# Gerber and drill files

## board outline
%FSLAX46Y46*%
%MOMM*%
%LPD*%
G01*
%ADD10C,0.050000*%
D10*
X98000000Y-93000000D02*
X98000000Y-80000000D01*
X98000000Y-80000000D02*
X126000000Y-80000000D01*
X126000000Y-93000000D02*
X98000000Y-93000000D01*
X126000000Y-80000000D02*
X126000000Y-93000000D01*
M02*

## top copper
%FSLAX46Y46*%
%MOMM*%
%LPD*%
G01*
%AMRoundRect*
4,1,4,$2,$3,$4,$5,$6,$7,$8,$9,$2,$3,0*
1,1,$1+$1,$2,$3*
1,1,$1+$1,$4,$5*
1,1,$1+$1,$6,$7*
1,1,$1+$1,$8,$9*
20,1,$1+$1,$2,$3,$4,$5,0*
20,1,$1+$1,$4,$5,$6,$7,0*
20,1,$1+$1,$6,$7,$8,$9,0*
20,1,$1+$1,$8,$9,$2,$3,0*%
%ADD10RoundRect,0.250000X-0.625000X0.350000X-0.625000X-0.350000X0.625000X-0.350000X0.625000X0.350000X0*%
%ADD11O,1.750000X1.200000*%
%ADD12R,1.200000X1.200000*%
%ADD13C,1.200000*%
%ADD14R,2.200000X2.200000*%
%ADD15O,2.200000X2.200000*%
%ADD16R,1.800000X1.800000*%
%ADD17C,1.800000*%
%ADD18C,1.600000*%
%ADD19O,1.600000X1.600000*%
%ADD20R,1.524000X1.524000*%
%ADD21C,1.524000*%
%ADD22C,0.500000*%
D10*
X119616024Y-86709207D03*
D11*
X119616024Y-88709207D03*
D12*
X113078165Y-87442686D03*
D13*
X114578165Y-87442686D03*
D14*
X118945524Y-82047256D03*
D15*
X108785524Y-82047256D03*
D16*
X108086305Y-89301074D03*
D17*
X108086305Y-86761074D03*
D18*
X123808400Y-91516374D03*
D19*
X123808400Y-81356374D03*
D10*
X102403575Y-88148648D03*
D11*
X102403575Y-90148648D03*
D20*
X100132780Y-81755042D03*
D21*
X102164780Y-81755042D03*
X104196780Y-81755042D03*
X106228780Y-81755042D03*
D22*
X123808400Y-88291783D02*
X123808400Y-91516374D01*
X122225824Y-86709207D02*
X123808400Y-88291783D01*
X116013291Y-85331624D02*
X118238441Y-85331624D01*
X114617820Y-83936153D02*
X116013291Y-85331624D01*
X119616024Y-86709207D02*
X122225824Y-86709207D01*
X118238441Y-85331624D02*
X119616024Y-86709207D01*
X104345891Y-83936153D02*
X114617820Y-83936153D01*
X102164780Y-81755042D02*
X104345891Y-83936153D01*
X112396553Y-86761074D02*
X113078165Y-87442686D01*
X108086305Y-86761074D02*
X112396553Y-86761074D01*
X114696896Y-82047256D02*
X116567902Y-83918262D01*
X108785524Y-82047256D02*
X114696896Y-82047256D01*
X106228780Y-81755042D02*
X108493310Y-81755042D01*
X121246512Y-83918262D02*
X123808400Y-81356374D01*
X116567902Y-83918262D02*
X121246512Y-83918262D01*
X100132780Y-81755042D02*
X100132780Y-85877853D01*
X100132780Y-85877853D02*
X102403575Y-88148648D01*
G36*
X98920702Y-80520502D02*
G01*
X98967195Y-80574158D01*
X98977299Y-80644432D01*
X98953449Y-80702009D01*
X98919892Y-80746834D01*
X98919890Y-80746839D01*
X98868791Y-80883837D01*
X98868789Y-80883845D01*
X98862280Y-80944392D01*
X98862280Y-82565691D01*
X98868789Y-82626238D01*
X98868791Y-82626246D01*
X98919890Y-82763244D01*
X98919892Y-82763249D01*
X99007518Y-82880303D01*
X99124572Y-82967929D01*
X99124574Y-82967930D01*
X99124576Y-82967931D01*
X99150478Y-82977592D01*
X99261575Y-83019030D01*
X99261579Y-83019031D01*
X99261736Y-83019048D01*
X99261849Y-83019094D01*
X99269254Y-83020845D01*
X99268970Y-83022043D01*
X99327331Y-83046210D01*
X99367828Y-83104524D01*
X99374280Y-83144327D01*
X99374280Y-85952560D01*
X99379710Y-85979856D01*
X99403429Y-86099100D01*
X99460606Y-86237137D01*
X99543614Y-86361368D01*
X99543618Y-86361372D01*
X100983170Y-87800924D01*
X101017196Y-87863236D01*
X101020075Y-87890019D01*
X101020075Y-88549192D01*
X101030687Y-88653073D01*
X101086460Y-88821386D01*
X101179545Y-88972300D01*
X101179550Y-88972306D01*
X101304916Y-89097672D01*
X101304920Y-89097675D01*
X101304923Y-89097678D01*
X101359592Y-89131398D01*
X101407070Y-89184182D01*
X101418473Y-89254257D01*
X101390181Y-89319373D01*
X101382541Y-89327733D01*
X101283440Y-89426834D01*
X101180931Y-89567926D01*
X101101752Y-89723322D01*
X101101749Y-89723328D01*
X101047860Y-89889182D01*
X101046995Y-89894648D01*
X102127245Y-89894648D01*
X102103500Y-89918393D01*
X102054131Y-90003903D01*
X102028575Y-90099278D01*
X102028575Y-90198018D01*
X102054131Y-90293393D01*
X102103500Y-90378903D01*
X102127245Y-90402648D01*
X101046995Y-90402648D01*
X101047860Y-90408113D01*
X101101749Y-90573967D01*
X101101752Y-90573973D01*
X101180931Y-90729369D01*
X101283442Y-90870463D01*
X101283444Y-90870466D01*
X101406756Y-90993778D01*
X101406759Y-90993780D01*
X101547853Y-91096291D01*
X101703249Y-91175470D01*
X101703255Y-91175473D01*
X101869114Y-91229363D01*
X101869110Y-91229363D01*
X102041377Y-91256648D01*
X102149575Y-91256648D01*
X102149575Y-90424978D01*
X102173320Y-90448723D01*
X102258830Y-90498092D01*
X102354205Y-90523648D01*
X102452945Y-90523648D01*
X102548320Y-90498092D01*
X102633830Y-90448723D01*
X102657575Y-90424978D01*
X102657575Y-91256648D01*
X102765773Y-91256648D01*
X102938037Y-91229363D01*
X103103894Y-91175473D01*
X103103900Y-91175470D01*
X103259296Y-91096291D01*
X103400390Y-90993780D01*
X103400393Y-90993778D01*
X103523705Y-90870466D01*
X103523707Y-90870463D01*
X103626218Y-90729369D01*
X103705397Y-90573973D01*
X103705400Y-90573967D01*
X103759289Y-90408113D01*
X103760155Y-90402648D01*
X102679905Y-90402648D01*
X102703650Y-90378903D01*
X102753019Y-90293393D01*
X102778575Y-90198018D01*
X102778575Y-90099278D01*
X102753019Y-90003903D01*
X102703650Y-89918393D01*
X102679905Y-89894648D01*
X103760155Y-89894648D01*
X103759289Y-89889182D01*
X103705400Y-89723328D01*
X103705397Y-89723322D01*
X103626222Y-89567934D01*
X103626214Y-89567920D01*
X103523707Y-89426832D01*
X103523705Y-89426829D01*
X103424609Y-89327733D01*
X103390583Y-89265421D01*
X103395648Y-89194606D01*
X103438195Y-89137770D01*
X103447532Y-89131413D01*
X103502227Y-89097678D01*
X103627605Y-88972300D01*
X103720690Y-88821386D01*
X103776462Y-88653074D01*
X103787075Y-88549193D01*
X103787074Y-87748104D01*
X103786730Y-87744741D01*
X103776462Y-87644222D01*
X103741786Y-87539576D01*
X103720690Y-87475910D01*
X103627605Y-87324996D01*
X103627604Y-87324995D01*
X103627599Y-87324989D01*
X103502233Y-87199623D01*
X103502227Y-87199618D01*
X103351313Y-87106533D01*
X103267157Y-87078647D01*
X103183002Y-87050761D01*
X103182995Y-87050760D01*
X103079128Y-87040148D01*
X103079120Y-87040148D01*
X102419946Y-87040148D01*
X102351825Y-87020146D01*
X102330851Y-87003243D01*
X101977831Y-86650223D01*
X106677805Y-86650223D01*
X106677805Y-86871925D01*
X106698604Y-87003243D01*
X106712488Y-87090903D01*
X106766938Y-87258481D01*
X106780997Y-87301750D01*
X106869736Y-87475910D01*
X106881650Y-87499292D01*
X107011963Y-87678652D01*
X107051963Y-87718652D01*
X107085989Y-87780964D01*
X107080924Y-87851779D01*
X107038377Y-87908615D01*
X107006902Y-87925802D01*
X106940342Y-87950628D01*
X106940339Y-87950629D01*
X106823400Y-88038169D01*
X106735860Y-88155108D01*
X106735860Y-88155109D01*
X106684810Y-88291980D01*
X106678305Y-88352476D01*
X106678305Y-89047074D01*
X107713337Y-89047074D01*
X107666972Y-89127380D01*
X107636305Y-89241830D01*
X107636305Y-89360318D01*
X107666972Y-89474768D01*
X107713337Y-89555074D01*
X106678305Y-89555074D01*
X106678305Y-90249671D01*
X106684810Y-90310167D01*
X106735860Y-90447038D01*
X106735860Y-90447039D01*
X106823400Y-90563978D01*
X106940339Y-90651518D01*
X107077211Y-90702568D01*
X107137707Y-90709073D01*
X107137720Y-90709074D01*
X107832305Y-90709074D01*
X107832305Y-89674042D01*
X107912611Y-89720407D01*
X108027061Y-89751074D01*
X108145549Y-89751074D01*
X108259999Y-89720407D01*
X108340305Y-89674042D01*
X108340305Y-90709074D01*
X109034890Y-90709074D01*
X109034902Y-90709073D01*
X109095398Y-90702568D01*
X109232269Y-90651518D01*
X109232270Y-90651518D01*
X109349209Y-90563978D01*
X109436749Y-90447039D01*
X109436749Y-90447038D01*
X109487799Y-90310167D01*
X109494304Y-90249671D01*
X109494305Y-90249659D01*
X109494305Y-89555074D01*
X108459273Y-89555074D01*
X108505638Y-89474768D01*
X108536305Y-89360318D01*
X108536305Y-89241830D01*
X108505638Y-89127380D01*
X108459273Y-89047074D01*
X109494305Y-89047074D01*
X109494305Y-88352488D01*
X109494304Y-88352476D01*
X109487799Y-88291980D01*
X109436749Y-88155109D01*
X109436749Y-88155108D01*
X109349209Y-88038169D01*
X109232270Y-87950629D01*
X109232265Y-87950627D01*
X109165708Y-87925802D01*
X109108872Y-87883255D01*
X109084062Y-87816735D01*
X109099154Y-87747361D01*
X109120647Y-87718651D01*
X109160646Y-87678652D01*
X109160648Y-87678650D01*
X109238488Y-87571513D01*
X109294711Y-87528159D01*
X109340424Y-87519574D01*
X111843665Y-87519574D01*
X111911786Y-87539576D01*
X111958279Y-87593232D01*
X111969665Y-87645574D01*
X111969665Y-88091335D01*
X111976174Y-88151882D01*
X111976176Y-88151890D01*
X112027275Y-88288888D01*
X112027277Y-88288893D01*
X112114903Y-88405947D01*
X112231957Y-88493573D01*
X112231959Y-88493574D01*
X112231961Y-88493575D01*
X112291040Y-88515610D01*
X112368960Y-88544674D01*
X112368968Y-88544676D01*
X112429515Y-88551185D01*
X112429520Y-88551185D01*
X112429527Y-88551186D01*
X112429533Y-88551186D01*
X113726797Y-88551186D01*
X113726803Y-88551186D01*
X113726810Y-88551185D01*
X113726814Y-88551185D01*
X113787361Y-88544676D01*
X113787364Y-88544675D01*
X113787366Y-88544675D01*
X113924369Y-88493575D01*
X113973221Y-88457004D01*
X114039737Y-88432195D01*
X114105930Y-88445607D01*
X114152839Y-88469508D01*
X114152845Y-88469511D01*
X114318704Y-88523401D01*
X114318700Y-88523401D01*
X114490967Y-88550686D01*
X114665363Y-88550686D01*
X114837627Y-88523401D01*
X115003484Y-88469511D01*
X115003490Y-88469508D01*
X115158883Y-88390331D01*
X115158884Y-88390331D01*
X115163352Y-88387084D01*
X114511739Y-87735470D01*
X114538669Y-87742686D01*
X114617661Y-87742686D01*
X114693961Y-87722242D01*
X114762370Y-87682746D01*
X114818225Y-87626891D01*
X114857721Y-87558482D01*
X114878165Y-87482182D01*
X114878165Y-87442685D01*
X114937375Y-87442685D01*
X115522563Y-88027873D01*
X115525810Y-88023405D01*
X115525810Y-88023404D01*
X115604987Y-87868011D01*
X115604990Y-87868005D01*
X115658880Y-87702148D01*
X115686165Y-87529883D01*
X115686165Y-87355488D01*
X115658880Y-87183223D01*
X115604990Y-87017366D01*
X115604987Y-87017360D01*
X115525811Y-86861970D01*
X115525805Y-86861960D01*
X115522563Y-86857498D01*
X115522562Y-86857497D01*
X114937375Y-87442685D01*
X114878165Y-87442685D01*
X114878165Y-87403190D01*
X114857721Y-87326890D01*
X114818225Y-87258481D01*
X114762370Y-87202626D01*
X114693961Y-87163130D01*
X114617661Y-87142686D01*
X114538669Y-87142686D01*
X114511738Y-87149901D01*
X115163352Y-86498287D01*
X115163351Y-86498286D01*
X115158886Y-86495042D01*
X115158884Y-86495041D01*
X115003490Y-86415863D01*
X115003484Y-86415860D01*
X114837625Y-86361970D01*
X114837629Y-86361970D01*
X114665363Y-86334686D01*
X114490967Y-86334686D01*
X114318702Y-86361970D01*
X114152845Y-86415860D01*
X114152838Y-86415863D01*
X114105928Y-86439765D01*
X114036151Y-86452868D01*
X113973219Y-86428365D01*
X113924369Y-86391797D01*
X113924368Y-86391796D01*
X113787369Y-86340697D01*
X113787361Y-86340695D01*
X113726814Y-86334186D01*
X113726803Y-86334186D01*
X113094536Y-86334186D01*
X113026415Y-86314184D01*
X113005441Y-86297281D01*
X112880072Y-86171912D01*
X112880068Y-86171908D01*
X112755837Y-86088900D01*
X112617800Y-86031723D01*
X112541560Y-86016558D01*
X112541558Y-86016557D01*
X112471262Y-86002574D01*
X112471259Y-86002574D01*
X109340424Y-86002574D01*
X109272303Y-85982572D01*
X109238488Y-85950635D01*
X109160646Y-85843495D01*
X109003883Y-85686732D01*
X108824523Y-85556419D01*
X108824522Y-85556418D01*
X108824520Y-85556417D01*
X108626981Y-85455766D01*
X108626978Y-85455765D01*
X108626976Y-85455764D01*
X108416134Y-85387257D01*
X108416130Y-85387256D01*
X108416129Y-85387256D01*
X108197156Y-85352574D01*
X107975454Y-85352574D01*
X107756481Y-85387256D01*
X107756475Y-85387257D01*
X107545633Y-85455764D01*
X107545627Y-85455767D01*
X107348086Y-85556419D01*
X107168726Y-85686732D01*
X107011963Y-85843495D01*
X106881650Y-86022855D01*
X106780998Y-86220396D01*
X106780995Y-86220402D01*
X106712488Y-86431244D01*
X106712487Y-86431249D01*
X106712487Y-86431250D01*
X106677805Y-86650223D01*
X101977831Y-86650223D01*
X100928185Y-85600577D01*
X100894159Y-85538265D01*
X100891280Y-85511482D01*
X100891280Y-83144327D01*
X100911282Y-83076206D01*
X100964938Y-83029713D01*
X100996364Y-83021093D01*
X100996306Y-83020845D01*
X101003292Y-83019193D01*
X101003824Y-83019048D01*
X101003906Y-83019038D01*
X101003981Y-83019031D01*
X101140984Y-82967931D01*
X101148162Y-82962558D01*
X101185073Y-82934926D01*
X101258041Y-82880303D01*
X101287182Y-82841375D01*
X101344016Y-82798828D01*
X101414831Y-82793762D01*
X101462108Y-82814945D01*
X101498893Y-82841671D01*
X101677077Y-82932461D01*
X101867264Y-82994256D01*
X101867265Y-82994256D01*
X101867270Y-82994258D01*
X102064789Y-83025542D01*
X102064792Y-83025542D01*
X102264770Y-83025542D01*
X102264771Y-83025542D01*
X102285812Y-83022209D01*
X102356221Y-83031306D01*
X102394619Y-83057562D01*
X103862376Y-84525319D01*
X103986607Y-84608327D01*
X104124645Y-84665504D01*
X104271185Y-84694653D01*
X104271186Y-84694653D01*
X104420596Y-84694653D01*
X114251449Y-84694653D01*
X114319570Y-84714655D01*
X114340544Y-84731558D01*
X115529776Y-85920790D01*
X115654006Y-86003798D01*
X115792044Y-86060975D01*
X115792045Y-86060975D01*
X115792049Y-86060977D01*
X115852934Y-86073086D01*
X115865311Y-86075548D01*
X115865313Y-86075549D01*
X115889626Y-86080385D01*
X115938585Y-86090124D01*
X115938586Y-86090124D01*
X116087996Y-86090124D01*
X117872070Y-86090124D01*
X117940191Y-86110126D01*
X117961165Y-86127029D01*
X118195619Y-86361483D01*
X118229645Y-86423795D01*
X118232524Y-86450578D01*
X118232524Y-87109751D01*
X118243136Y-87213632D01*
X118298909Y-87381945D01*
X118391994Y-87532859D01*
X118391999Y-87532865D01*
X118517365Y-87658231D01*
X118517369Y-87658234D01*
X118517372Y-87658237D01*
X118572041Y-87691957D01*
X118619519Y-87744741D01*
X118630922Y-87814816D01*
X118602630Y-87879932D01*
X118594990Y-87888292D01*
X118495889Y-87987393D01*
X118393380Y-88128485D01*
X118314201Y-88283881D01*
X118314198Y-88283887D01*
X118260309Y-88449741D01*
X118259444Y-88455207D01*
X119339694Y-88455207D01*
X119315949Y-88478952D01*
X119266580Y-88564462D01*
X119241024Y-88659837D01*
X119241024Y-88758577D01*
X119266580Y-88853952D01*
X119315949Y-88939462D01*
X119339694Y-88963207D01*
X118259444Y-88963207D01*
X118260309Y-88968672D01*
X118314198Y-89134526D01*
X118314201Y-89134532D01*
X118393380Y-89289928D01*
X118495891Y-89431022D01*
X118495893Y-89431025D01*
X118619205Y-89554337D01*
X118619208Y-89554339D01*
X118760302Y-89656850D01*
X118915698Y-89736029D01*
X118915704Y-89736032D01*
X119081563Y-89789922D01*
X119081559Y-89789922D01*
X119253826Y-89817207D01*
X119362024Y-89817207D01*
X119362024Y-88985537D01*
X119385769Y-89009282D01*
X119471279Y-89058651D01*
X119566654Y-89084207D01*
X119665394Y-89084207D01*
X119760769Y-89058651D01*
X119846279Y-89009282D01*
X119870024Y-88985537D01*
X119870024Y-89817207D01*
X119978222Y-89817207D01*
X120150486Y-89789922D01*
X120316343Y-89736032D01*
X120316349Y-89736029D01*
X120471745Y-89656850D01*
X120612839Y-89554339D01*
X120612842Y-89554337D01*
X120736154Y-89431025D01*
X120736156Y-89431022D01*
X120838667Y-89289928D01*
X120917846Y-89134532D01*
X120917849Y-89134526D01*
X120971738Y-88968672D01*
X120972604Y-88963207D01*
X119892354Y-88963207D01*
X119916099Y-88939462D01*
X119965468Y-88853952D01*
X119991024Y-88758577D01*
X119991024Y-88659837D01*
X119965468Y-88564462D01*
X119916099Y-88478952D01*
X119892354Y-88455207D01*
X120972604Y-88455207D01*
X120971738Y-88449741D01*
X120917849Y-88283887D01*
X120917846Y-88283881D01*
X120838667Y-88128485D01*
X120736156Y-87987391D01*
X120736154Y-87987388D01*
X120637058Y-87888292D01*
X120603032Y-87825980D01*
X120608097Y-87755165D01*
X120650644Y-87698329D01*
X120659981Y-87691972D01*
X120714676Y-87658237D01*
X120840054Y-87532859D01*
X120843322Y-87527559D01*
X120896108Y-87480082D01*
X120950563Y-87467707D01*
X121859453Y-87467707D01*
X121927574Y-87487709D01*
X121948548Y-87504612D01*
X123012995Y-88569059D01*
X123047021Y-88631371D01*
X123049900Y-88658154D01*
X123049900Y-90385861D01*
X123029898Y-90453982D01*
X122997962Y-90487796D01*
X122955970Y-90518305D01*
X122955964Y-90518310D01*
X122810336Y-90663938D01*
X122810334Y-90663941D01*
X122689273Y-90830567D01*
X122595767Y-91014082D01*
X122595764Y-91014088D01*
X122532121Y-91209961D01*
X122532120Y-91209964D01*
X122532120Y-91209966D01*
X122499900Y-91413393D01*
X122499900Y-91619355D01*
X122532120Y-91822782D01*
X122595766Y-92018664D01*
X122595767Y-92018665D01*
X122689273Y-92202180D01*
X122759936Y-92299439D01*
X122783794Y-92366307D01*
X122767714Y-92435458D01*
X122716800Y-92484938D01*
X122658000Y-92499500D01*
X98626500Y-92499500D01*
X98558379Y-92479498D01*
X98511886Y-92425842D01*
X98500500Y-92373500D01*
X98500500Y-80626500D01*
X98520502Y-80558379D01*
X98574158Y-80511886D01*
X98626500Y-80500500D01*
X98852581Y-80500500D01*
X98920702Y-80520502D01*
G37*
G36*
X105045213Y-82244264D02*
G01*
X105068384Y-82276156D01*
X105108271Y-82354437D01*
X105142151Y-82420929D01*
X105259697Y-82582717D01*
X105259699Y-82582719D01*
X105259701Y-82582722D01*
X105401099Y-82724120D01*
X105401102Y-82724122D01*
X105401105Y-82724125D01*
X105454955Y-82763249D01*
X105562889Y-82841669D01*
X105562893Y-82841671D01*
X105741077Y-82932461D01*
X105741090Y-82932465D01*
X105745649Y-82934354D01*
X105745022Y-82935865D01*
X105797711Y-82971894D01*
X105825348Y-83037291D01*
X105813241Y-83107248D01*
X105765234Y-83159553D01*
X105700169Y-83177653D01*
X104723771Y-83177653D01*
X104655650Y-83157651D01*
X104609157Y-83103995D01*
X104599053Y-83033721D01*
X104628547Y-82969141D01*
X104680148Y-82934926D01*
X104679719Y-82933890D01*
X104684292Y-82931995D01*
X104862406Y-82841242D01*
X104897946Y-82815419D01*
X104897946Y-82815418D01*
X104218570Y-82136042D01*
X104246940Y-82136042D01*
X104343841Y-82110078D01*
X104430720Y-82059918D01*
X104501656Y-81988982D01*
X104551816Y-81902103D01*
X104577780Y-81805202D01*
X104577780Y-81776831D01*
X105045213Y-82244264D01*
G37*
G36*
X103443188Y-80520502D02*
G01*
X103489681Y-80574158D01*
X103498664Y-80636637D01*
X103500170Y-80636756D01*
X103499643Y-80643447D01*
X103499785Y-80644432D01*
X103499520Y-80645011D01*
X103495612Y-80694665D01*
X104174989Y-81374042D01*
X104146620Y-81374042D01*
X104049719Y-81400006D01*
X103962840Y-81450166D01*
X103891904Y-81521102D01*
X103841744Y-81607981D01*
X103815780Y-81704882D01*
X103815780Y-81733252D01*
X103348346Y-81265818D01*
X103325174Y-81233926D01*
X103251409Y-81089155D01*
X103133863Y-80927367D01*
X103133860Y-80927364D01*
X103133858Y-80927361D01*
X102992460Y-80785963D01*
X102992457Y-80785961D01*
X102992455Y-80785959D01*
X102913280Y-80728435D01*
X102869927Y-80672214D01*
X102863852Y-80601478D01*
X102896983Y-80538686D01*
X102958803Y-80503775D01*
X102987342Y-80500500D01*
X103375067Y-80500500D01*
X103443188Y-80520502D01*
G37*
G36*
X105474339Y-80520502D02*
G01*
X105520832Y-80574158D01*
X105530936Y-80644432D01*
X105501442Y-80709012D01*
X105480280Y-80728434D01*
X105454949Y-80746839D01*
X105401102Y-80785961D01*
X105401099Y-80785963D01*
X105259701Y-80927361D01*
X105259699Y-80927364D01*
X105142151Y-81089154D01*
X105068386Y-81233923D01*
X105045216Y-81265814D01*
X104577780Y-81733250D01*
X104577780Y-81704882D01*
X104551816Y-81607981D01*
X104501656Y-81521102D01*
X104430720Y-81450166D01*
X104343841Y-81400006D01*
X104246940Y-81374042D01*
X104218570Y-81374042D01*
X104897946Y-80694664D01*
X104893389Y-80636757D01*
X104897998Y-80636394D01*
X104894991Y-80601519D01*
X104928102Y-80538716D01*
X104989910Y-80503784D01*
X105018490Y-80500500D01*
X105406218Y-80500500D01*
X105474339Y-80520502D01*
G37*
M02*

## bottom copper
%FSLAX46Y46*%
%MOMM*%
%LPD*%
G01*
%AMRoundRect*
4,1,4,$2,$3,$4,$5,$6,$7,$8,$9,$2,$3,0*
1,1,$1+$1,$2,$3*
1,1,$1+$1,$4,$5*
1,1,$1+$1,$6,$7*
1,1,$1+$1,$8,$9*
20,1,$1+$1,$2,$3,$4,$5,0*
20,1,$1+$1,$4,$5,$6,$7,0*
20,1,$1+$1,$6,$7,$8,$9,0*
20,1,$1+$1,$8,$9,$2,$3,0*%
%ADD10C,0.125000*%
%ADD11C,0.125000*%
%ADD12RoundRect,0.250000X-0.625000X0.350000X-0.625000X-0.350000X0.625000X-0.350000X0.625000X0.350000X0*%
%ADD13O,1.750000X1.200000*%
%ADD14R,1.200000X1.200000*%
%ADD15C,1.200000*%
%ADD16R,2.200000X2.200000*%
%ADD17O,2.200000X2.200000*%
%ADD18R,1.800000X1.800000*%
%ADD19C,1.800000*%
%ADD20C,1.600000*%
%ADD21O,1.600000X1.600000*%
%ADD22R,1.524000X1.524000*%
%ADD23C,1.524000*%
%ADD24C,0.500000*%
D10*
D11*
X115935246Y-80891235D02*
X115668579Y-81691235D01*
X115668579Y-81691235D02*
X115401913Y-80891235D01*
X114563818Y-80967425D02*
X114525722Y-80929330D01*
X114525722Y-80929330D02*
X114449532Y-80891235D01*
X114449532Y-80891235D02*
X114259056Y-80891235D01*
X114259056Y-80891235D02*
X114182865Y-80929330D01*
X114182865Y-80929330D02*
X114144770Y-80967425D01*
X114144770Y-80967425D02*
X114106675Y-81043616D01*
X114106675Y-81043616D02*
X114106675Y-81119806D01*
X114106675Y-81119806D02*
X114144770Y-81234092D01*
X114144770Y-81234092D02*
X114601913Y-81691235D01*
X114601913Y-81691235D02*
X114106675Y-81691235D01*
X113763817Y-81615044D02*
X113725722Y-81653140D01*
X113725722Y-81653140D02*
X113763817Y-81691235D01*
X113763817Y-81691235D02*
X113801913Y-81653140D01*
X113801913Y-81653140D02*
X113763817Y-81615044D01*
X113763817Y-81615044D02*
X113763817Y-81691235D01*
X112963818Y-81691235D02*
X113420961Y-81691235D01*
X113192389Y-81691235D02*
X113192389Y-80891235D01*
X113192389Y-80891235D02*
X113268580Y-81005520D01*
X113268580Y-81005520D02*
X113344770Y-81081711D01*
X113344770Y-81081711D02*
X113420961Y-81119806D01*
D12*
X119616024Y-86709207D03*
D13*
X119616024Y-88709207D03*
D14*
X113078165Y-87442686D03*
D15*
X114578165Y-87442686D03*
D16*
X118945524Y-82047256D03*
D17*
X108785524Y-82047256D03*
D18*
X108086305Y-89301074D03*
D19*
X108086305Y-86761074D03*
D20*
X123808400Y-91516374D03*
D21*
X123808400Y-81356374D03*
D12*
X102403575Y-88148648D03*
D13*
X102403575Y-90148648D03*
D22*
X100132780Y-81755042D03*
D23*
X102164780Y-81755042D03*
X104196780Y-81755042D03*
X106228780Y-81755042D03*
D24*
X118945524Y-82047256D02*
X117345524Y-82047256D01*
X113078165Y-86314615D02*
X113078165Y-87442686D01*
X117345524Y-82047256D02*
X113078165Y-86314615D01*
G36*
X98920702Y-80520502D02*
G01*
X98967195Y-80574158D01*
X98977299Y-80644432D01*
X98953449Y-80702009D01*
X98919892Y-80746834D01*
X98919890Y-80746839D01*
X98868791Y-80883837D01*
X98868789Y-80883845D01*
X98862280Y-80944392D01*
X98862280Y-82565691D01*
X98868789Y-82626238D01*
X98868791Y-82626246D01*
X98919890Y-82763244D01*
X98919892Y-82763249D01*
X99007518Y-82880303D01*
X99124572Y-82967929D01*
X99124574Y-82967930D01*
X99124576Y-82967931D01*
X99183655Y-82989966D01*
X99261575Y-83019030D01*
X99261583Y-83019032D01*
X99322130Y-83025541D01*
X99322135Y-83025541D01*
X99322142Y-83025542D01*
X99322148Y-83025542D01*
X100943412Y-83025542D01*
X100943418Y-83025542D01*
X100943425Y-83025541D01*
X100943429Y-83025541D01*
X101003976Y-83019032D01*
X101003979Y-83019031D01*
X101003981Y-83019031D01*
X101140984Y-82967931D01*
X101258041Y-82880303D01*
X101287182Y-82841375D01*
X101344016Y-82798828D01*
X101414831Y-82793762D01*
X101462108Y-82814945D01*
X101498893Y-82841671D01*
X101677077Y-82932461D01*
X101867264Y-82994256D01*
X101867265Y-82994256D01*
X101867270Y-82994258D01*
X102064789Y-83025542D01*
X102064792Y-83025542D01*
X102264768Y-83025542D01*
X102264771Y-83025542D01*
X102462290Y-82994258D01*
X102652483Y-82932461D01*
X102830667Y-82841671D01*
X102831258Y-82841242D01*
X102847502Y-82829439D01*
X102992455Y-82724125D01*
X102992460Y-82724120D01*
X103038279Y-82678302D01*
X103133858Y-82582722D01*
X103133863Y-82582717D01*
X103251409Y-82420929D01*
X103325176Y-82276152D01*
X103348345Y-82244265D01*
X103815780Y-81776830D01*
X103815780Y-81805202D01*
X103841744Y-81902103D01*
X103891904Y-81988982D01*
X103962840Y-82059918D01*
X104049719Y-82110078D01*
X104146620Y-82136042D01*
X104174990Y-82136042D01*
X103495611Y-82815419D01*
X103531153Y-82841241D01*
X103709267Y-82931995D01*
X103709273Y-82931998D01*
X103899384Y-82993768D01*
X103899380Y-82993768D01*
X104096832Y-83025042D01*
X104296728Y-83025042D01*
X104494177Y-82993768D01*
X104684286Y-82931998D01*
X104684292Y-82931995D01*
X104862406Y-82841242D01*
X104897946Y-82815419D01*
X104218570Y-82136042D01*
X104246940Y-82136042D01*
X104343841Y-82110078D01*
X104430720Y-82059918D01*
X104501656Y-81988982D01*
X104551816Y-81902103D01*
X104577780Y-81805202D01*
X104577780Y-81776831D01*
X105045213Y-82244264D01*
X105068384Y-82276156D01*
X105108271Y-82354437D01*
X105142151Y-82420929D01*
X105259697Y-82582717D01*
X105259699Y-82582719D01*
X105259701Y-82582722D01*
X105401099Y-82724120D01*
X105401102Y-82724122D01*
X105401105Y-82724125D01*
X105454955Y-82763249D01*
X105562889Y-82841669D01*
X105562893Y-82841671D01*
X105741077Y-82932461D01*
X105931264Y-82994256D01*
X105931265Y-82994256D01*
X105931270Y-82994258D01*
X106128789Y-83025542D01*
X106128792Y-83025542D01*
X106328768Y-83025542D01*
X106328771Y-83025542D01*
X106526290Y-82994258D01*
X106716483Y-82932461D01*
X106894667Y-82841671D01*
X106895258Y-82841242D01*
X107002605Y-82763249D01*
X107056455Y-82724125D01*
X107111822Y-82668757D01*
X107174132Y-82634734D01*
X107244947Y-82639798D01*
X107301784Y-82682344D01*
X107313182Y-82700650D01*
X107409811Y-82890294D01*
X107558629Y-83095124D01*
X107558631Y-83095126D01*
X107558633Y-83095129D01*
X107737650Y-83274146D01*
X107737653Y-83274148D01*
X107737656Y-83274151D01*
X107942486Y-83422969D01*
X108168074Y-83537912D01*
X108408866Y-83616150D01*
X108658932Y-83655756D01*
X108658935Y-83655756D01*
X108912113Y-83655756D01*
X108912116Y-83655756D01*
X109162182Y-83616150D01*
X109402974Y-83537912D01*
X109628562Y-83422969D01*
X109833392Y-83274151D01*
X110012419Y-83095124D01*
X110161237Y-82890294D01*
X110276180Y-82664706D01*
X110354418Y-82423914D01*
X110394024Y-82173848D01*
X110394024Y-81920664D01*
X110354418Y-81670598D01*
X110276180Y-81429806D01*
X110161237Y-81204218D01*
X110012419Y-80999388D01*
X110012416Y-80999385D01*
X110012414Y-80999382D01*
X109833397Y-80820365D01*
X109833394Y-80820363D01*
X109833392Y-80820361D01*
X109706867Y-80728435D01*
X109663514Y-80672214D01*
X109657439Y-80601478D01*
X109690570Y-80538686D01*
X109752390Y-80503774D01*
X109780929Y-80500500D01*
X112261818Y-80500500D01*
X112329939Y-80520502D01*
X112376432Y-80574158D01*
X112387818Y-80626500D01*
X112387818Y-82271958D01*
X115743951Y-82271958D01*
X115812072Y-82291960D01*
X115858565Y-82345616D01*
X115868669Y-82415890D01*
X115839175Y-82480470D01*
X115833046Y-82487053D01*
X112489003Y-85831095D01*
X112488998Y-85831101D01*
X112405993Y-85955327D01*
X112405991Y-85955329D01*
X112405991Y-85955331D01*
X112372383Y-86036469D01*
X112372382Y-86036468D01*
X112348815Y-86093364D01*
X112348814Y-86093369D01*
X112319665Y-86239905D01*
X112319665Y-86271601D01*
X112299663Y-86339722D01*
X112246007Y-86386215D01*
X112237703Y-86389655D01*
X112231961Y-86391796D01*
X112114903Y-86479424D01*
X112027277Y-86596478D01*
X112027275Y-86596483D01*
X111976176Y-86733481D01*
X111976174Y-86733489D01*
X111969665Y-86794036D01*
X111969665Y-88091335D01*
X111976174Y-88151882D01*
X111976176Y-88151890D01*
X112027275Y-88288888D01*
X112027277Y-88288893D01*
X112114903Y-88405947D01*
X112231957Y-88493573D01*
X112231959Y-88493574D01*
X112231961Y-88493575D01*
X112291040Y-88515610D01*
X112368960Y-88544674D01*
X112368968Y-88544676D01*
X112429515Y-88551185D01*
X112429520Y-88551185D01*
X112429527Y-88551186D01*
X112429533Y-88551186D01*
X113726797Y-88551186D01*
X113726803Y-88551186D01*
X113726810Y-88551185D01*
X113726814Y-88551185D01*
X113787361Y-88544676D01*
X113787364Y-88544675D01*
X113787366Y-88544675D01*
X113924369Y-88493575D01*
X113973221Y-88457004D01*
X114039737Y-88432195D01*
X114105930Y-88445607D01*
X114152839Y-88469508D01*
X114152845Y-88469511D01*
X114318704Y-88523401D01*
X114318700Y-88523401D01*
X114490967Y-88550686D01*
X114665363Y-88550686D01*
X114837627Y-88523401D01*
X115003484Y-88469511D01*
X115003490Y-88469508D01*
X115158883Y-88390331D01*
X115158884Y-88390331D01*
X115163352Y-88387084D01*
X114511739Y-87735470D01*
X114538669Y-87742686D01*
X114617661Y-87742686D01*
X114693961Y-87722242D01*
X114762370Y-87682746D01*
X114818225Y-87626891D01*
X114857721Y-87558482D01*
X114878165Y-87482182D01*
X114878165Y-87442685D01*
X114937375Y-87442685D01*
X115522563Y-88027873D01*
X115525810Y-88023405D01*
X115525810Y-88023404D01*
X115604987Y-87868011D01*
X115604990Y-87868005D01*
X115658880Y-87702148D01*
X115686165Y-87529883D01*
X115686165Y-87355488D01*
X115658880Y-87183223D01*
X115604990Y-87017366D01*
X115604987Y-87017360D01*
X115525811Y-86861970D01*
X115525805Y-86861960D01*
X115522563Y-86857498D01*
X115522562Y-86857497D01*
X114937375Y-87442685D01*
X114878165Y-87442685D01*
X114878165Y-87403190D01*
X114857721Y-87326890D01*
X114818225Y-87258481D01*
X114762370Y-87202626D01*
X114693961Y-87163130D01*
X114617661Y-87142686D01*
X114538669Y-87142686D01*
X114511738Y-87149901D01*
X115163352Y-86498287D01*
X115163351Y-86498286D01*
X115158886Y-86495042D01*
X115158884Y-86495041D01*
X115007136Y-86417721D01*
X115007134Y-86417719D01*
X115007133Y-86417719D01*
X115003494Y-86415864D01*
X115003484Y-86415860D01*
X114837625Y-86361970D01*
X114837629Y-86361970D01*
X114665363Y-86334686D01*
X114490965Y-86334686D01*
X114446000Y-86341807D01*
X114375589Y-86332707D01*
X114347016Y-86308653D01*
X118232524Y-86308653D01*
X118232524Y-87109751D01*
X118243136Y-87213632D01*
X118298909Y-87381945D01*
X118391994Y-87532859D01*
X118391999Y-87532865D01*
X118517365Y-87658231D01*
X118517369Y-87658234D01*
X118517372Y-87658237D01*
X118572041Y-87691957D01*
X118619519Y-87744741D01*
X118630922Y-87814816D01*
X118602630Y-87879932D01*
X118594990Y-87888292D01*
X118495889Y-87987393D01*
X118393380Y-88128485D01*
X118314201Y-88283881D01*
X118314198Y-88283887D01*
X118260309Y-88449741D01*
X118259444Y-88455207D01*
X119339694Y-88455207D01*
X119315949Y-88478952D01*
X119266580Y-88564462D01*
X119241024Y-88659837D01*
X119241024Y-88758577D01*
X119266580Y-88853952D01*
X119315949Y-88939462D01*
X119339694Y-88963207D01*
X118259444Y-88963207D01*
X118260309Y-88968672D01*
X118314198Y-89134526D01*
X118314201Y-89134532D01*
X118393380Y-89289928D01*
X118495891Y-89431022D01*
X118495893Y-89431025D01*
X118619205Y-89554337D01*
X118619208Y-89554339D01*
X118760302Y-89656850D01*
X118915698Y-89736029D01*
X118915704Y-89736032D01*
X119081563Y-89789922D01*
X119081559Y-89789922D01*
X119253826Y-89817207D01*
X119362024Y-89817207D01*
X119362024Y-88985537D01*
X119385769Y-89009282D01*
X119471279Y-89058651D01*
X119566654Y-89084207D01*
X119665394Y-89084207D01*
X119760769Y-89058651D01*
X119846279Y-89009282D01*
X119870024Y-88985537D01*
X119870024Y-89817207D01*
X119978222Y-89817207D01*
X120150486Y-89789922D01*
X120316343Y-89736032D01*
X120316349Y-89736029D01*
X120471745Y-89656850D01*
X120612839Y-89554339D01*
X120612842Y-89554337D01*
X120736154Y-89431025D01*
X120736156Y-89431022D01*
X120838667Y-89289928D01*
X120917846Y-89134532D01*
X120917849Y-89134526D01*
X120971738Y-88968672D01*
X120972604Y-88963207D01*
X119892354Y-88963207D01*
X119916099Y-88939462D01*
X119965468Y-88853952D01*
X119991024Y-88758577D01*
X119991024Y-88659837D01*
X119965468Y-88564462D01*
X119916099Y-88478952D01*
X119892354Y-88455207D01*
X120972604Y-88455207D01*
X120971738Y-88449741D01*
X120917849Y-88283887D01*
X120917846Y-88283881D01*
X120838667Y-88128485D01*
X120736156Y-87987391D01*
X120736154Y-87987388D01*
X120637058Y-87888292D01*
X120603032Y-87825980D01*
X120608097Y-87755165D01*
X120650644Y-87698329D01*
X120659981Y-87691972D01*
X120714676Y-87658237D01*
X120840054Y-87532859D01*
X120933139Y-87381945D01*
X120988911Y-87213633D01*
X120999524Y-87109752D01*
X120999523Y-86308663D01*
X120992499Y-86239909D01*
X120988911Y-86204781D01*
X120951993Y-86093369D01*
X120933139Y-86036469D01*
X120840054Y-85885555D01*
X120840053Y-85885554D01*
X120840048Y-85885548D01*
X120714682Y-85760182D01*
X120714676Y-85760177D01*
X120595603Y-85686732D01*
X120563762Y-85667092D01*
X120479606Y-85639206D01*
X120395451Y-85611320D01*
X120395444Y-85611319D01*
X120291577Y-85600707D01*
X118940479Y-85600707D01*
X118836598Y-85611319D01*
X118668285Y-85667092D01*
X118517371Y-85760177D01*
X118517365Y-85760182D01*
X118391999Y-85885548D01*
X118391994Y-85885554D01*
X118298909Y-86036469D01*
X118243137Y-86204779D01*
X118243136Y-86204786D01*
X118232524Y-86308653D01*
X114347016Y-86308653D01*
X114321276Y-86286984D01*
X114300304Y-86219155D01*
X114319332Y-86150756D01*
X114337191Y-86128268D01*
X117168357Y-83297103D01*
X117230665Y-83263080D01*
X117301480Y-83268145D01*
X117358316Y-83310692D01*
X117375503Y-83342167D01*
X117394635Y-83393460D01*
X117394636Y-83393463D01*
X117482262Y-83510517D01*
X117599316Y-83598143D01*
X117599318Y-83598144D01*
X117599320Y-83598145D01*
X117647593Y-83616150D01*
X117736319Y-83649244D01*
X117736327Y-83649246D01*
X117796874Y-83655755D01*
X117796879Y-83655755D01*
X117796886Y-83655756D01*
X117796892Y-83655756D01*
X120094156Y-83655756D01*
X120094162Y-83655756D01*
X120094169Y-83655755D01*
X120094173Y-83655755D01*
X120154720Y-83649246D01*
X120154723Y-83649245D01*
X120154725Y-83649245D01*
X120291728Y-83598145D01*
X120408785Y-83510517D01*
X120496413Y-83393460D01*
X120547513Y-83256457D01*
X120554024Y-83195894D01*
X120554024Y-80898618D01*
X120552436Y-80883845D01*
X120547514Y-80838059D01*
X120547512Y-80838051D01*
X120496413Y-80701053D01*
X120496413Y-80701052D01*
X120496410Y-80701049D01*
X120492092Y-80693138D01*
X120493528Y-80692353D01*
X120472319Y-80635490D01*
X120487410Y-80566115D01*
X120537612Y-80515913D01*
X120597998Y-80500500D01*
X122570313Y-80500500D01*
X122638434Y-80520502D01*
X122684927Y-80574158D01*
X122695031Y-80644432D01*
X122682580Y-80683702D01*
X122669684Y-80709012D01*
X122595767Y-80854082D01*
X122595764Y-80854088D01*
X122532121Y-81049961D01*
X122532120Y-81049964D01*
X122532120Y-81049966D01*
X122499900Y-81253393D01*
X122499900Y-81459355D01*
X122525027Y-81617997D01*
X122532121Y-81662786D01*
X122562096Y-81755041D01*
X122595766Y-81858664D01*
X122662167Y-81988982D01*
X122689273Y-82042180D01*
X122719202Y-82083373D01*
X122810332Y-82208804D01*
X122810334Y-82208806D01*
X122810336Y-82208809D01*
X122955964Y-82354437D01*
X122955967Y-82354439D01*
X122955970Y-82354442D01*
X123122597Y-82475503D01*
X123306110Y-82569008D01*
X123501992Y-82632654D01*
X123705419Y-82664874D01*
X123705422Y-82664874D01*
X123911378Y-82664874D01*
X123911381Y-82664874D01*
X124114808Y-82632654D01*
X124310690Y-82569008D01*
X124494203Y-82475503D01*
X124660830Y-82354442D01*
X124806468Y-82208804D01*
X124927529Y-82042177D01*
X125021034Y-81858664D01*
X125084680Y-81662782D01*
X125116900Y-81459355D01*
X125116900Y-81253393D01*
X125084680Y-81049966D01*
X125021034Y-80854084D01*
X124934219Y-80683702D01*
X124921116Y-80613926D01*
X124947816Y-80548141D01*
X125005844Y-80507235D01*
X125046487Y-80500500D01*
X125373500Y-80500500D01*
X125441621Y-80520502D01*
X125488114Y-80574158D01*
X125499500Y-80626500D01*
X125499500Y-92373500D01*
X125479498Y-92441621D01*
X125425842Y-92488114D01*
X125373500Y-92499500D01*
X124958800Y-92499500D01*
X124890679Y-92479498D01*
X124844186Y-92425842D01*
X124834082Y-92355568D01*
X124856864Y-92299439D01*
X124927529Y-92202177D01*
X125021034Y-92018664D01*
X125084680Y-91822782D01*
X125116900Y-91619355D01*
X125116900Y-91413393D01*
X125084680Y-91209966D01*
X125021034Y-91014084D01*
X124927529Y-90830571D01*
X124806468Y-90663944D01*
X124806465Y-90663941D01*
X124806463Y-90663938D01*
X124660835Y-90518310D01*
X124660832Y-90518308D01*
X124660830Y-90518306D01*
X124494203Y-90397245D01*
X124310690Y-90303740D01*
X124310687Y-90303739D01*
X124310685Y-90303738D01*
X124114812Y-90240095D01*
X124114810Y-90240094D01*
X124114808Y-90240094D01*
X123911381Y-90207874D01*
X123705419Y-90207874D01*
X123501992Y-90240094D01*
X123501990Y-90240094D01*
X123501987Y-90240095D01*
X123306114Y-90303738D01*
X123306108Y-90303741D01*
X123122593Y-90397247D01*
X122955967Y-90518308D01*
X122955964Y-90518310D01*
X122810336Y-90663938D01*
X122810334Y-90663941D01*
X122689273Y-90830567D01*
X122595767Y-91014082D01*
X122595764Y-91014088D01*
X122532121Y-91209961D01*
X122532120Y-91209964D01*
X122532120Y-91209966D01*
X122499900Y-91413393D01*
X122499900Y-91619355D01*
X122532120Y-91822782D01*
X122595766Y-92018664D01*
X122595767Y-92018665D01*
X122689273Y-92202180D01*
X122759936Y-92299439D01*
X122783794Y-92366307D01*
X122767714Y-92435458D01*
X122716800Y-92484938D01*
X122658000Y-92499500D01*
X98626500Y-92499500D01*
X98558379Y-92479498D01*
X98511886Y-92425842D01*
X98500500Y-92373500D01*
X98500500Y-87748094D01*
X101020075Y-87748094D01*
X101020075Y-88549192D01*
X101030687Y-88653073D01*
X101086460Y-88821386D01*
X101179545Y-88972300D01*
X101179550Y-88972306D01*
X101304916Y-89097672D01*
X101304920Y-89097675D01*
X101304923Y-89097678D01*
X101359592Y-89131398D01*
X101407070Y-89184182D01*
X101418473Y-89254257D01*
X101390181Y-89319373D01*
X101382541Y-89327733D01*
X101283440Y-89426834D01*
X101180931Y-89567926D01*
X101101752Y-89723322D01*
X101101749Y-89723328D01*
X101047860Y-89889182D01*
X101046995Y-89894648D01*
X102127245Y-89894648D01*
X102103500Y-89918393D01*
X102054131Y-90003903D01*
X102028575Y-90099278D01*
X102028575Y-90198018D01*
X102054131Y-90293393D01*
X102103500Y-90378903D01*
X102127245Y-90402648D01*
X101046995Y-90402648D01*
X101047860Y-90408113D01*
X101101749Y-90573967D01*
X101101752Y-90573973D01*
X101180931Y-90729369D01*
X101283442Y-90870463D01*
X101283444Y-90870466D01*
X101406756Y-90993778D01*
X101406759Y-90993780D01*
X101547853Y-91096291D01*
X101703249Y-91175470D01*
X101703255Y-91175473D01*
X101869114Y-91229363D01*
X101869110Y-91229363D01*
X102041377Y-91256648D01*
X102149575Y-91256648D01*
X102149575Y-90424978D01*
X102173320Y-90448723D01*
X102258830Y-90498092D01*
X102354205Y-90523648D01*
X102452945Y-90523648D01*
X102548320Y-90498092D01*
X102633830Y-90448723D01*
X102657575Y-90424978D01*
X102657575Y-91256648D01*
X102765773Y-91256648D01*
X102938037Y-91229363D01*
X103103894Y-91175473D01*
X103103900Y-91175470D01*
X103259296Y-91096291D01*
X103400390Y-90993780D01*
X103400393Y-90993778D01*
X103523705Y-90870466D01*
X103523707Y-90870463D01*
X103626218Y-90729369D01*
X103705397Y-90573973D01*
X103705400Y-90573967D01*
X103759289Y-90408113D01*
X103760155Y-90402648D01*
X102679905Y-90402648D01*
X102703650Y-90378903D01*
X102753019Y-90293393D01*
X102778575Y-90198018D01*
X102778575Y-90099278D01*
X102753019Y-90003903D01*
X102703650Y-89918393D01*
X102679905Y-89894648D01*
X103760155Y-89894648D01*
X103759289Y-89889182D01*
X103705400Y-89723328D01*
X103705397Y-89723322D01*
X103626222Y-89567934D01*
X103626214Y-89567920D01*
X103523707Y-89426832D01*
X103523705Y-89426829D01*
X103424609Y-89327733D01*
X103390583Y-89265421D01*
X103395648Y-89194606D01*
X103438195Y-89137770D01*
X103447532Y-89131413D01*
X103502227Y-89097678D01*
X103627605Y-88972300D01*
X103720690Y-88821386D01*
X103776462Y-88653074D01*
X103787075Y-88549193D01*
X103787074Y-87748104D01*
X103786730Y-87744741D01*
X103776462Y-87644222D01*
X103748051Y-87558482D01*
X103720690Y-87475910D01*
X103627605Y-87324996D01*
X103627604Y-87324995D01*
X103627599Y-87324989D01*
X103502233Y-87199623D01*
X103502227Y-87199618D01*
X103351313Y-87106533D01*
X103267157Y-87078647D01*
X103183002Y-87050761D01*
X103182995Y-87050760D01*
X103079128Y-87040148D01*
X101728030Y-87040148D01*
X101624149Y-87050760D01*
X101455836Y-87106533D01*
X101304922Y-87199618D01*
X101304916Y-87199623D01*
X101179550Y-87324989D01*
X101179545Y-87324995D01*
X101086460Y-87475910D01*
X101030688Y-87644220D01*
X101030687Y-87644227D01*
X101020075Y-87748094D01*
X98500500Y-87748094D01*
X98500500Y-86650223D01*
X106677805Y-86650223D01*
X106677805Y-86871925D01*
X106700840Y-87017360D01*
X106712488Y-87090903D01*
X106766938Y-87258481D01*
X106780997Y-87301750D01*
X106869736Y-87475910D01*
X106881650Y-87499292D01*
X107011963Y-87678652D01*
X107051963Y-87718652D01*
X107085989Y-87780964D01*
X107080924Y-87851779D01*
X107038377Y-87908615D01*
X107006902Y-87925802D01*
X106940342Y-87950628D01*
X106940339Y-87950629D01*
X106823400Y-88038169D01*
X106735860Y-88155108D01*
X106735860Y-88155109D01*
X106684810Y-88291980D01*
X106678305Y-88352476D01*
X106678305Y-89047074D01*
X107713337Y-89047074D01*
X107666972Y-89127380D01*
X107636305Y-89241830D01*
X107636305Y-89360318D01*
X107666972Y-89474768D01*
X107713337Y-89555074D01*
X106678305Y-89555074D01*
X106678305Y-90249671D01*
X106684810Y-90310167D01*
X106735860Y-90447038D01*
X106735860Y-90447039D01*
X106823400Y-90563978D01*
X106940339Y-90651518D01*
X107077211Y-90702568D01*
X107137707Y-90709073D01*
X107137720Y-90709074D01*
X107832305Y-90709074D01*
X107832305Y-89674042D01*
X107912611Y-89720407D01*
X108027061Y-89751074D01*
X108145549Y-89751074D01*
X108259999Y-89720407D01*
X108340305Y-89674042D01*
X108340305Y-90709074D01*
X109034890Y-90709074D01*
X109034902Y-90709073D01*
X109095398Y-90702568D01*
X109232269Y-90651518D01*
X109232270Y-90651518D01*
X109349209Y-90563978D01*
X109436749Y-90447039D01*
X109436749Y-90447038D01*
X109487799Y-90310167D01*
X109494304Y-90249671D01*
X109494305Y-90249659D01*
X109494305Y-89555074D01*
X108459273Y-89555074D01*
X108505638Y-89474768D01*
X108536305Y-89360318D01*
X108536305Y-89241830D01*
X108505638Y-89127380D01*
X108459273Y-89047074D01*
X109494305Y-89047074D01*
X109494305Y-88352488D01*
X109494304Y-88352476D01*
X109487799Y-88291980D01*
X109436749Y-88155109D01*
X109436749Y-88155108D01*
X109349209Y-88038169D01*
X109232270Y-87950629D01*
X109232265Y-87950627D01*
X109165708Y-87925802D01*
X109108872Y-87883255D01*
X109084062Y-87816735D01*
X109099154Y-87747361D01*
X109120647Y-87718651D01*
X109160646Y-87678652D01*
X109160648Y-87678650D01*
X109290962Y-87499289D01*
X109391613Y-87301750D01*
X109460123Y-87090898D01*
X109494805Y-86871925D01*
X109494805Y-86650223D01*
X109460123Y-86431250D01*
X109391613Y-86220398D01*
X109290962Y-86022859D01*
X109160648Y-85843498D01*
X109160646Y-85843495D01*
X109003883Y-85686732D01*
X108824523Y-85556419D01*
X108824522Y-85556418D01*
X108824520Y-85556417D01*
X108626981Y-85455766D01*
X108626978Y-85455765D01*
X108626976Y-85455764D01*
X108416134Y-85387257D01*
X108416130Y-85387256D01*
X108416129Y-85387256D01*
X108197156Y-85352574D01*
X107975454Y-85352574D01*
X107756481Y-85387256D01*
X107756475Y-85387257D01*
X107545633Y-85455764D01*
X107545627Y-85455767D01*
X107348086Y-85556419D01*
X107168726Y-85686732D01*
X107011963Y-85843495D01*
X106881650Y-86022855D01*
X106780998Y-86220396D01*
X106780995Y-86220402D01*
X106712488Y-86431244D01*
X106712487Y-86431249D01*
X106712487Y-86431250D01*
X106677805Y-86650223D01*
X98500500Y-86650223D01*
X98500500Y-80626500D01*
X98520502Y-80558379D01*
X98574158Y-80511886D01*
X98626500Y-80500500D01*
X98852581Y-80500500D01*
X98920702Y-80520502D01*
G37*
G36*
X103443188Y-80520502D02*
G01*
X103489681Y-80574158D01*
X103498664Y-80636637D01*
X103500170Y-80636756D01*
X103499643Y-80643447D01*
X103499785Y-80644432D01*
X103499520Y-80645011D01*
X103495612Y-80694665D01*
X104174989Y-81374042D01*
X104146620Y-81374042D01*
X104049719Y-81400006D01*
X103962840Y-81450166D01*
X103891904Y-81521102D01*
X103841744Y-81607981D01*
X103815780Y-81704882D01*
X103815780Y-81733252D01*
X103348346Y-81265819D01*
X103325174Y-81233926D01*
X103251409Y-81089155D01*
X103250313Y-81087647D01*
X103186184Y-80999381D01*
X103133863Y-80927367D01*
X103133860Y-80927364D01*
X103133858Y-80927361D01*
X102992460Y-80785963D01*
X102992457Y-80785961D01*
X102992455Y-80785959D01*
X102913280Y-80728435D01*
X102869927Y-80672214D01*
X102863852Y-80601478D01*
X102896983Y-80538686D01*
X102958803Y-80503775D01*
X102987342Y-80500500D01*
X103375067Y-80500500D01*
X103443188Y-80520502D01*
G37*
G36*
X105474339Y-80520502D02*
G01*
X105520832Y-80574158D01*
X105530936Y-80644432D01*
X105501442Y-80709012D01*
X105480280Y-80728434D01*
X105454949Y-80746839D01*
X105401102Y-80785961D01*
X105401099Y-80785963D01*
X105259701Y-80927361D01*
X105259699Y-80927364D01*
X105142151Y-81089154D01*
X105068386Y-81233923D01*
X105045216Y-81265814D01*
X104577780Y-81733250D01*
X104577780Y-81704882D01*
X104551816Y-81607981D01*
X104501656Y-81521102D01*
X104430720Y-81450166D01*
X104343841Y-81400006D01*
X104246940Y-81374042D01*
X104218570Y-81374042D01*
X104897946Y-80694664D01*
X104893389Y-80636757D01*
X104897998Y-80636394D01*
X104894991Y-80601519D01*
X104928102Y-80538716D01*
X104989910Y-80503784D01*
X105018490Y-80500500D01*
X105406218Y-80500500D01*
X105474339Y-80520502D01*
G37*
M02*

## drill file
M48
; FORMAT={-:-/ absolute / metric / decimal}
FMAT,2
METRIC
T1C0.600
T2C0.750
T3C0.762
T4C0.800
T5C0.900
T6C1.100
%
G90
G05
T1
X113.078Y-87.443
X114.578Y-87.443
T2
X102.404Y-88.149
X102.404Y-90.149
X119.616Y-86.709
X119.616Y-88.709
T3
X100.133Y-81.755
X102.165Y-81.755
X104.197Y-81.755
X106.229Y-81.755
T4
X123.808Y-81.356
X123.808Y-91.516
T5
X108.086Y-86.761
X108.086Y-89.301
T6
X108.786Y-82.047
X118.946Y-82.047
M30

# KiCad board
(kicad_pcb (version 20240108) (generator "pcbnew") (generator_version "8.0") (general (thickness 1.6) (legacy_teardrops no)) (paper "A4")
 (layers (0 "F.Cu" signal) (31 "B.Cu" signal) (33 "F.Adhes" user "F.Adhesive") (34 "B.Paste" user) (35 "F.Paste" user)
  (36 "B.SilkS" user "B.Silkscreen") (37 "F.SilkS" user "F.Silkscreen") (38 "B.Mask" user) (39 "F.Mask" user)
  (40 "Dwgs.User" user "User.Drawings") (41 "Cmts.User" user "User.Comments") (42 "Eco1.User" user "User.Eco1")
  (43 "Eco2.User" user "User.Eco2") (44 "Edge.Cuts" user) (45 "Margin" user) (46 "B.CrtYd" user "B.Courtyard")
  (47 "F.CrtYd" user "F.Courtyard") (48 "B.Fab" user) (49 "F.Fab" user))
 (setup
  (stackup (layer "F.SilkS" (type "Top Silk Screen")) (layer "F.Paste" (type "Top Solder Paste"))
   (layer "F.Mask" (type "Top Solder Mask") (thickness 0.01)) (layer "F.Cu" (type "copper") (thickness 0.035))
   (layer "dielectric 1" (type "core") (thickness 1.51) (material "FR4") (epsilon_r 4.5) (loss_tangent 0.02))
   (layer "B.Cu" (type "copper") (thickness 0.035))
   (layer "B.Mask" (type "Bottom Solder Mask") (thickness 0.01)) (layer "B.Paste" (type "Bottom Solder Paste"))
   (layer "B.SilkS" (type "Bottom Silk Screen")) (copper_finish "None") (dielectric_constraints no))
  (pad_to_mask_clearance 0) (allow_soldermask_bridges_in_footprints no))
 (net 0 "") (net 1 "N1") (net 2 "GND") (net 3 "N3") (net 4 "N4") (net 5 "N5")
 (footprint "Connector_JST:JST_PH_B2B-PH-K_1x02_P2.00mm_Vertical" (layer "F.Cu") (at 119.616024 86.709207 -90)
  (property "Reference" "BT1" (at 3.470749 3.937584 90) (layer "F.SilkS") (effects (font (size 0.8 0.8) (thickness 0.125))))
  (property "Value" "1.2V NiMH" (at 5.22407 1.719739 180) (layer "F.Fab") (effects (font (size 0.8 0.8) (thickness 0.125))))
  (pad "1" thru_hole roundrect (at 0 0 270) (size 1.2 1.75) (drill 0.75) (layers "*.Cu" "*.Mask") (remove_unused_layers no)
   (roundrect_rratio 0.2083333333) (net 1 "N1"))
  (pad "2" thru_hole oval (at 2 0 270) (size 1.2 1.75) (drill 0.75) (layers "*.Cu" "*.Mask") (remove_unused_layers no) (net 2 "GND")))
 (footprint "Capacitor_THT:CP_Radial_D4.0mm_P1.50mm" (layer "F.Cu") (at 113.078165 87.442686)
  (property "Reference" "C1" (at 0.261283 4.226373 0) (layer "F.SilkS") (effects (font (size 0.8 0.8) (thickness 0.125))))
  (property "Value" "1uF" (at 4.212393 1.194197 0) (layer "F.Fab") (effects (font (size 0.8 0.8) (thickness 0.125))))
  (pad "1" thru_hole rect (at 0 0) (size 1.2 1.2) (drill 0.6) (layers "*.Cu" "*.Mask") (remove_unused_layers no) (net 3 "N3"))
  (pad "2" thru_hole circle (at 1.5 0) (size 1.2 1.2) (drill 0.6) (layers "*.Cu" "*.Mask") (remove_unused_layers no) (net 2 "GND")))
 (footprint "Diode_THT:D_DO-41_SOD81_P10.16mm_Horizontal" (layer "F.Cu") (at 118.945524 82.047256 180)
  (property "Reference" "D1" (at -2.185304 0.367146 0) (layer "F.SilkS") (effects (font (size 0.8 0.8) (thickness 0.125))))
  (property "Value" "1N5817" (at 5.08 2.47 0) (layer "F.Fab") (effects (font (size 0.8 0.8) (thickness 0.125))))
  (pad "1" thru_hole rect (at 0 0 180) (size 2.2 2.2) (drill 1.1) (layers "*.Cu" "*.Mask") (remove_unused_layers no) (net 3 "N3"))
  (pad "2" thru_hole oval (at 10.16 0 180) (size 2.2 2.2) (drill 1.1) (layers "*.Cu" "*.Mask") (remove_unused_layers no) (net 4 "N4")))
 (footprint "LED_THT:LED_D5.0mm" (layer "F.Cu") (at 108.086305 89.301074 90)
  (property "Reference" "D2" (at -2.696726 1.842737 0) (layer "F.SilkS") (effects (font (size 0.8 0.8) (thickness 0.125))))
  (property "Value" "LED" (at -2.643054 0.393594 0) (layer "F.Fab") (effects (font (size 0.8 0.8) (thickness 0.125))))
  (pad "1" thru_hole rect (at 0 0 90) (size 1.8 1.8) (drill 0.9) (layers "*.Cu" "*.Mask") (remove_unused_layers no) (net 2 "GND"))
  (pad "2" thru_hole circle (at 2.54 0 90) (size 1.8 1.8) (drill 0.9) (layers "*.Cu" "*.Mask") (remove_unused_layers no) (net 3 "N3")))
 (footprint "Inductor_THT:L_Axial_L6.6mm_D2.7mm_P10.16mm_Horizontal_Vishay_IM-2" (layer "F.Cu") (at 123.8084 91.516374 90)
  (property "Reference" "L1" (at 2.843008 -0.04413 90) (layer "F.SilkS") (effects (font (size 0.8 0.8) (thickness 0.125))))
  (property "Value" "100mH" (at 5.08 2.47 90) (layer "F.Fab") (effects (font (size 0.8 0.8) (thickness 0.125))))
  (pad "1" thru_hole circle (at 0 0 90) (size 1.6 1.6) (drill 0.8) (layers "*.Cu" "*.Mask") (remove_unused_layers no) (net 1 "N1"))
  (pad "2" thru_hole oval (at 10.16 0 90) (size 1.6 1.6) (drill 0.8) (layers "*.Cu" "*.Mask") (remove_unused_layers no) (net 4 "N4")))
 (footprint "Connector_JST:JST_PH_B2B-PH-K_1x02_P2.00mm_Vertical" (layer "F.Cu") (at 102.403575 88.148648 -90)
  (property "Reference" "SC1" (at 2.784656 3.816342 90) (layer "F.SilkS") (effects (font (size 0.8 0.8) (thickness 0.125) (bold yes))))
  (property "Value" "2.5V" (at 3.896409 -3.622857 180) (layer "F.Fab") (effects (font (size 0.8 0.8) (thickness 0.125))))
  (pad "1" thru_hole roundrect (at 0 0 270) (size 1.2 1.75) (drill 0.75) (layers "*.Cu" "*.Mask") (remove_unused_layers no)
   (roundrect_rratio 0.2083333333) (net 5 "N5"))
  (pad "2" thru_hole oval (at 2 0 270) (size 1.2 1.75) (drill 0.75) (layers "*.Cu" "*.Mask") (remove_unused_layers no) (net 2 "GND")))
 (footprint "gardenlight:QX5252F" (layer "F.Cu") (at 103.18078 81.755042)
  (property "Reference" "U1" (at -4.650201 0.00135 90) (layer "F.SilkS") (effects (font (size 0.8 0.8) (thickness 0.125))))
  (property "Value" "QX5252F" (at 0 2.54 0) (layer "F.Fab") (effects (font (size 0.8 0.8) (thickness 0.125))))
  (pad "1" thru_hole rect (at -3.048 0) (size 1.524 1.524) (drill 0.762) (layers "*.Cu" "*.Mask") (remove_unused_layers no) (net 5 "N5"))
  (pad "2" thru_hole circle (at -1.016 0) (size 1.524 1.524) (drill 0.762) (layers "*.Cu" "*.Mask") (remove_unused_layers no) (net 1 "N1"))
  (pad "3" thru_hole circle (at 1.016 0) (size 1.524 1.524) (drill 0.762) (layers "*.Cu" "*.Mask") (remove_unused_layers no) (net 2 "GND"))
  (pad "4" thru_hole circle (at 3.048 0) (size 1.524 1.524) (drill 0.762) (layers "*.Cu" "*.Mask") (remove_unused_layers no) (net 4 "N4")))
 (gr_line (start 98 93) (end 98 80) (stroke (width 0.05) (type solid)) (layer "Edge.Cuts"))
 (gr_line (start 98 80) (end 126 80) (stroke (width 0.05) (type solid)) (layer "Edge.Cuts"))
 (gr_line (start 126 93) (end 98 93) (stroke (width 0.05) (type solid)) (layer "Edge.Cuts"))
 (gr_line (start 126 80) (end 126 93) (stroke (width 0.05) (type solid)) (layer "Edge.Cuts"))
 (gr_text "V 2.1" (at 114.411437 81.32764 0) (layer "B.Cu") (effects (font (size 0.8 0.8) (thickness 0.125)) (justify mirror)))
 (segment (start 123.8084 88.291783) (end 123.8084 91.516374) (width 0.5) (layer "F.Cu") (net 1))
 (segment (start 122.225824 86.709207) (end 123.8084 88.291783) (width 0.5) (layer "F.Cu") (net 1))
 (segment (start 116.013291 85.331624) (end 118.238441 85.331624) (width 0.5) (layer "F.Cu") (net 1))
 (segment (start 114.61782 83.936153) (end 116.013291 85.331624) (width 0.5) (layer "F.Cu") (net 1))
 (segment (start 119.616024 86.709207) (end 122.225824 86.709207) (width 0.5) (layer "F.Cu") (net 1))
 (segment (start 118.238441 85.331624) (end 119.616024 86.709207) (width 0.5) (layer "F.Cu") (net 1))
 (segment (start 104.345891 83.936153) (end 114.61782 83.936153) (width 0.5) (layer "F.Cu") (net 1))
 (segment (start 102.16478 81.755042) (end 104.345891 83.936153) (width 0.5) (layer "F.Cu") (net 1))
 (segment (start 112.396553 86.761074) (end 113.078165 87.442686) (width 0.5) (layer "F.Cu") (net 3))
 (segment (start 108.086305 86.761074) (end 112.396553 86.761074) (width 0.5) (layer "F.Cu") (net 3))
 (segment (start 118.945524 82.047256) (end 117.345524 82.047256) (width 0.5) (layer "B.Cu") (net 3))
 (segment (start 113.078165 86.314615) (end 113.078165 87.442686) (width 0.5) (layer "B.Cu") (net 3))
 (segment (start 117.345524 82.047256) (end 113.078165 86.314615) (width 0.5) (layer "B.Cu") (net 3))
 (segment (start 114.696896 82.047256) (end 116.567902 83.918262) (width 0.5) (layer "F.Cu") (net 4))
 (segment (start 108.785524 82.047256) (end 114.696896 82.047256) (width 0.5) (layer "F.Cu") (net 4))
 (segment (start 106.22878 81.755042) (end 108.49331 81.755042) (width 0.5) (layer "F.Cu") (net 4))
 (segment (start 121.246512 83.918262) (end 123.8084 81.356374) (width 0.5) (layer "F.Cu") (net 4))
 (segment (start 116.567902 83.918262) (end 121.246512 83.918262) (width 0.5) (layer "F.Cu") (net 4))
 (segment (start 100.13278 81.755042) (end 100.13278 85.877853) (width 0.5) (layer "F.Cu") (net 5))
 (segment (start 100.13278 85.877853) (end 102.403575 88.148648) (width 0.5) (layer "F.Cu") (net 5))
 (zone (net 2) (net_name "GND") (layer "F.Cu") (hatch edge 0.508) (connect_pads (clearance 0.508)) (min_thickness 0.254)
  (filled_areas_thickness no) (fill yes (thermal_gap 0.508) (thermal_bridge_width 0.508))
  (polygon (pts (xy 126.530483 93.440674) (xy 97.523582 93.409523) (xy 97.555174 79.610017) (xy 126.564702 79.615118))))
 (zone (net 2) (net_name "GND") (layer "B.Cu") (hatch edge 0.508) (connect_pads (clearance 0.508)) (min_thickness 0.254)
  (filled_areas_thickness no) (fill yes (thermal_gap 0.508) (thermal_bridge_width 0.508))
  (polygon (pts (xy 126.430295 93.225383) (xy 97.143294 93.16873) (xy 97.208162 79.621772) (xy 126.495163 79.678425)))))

